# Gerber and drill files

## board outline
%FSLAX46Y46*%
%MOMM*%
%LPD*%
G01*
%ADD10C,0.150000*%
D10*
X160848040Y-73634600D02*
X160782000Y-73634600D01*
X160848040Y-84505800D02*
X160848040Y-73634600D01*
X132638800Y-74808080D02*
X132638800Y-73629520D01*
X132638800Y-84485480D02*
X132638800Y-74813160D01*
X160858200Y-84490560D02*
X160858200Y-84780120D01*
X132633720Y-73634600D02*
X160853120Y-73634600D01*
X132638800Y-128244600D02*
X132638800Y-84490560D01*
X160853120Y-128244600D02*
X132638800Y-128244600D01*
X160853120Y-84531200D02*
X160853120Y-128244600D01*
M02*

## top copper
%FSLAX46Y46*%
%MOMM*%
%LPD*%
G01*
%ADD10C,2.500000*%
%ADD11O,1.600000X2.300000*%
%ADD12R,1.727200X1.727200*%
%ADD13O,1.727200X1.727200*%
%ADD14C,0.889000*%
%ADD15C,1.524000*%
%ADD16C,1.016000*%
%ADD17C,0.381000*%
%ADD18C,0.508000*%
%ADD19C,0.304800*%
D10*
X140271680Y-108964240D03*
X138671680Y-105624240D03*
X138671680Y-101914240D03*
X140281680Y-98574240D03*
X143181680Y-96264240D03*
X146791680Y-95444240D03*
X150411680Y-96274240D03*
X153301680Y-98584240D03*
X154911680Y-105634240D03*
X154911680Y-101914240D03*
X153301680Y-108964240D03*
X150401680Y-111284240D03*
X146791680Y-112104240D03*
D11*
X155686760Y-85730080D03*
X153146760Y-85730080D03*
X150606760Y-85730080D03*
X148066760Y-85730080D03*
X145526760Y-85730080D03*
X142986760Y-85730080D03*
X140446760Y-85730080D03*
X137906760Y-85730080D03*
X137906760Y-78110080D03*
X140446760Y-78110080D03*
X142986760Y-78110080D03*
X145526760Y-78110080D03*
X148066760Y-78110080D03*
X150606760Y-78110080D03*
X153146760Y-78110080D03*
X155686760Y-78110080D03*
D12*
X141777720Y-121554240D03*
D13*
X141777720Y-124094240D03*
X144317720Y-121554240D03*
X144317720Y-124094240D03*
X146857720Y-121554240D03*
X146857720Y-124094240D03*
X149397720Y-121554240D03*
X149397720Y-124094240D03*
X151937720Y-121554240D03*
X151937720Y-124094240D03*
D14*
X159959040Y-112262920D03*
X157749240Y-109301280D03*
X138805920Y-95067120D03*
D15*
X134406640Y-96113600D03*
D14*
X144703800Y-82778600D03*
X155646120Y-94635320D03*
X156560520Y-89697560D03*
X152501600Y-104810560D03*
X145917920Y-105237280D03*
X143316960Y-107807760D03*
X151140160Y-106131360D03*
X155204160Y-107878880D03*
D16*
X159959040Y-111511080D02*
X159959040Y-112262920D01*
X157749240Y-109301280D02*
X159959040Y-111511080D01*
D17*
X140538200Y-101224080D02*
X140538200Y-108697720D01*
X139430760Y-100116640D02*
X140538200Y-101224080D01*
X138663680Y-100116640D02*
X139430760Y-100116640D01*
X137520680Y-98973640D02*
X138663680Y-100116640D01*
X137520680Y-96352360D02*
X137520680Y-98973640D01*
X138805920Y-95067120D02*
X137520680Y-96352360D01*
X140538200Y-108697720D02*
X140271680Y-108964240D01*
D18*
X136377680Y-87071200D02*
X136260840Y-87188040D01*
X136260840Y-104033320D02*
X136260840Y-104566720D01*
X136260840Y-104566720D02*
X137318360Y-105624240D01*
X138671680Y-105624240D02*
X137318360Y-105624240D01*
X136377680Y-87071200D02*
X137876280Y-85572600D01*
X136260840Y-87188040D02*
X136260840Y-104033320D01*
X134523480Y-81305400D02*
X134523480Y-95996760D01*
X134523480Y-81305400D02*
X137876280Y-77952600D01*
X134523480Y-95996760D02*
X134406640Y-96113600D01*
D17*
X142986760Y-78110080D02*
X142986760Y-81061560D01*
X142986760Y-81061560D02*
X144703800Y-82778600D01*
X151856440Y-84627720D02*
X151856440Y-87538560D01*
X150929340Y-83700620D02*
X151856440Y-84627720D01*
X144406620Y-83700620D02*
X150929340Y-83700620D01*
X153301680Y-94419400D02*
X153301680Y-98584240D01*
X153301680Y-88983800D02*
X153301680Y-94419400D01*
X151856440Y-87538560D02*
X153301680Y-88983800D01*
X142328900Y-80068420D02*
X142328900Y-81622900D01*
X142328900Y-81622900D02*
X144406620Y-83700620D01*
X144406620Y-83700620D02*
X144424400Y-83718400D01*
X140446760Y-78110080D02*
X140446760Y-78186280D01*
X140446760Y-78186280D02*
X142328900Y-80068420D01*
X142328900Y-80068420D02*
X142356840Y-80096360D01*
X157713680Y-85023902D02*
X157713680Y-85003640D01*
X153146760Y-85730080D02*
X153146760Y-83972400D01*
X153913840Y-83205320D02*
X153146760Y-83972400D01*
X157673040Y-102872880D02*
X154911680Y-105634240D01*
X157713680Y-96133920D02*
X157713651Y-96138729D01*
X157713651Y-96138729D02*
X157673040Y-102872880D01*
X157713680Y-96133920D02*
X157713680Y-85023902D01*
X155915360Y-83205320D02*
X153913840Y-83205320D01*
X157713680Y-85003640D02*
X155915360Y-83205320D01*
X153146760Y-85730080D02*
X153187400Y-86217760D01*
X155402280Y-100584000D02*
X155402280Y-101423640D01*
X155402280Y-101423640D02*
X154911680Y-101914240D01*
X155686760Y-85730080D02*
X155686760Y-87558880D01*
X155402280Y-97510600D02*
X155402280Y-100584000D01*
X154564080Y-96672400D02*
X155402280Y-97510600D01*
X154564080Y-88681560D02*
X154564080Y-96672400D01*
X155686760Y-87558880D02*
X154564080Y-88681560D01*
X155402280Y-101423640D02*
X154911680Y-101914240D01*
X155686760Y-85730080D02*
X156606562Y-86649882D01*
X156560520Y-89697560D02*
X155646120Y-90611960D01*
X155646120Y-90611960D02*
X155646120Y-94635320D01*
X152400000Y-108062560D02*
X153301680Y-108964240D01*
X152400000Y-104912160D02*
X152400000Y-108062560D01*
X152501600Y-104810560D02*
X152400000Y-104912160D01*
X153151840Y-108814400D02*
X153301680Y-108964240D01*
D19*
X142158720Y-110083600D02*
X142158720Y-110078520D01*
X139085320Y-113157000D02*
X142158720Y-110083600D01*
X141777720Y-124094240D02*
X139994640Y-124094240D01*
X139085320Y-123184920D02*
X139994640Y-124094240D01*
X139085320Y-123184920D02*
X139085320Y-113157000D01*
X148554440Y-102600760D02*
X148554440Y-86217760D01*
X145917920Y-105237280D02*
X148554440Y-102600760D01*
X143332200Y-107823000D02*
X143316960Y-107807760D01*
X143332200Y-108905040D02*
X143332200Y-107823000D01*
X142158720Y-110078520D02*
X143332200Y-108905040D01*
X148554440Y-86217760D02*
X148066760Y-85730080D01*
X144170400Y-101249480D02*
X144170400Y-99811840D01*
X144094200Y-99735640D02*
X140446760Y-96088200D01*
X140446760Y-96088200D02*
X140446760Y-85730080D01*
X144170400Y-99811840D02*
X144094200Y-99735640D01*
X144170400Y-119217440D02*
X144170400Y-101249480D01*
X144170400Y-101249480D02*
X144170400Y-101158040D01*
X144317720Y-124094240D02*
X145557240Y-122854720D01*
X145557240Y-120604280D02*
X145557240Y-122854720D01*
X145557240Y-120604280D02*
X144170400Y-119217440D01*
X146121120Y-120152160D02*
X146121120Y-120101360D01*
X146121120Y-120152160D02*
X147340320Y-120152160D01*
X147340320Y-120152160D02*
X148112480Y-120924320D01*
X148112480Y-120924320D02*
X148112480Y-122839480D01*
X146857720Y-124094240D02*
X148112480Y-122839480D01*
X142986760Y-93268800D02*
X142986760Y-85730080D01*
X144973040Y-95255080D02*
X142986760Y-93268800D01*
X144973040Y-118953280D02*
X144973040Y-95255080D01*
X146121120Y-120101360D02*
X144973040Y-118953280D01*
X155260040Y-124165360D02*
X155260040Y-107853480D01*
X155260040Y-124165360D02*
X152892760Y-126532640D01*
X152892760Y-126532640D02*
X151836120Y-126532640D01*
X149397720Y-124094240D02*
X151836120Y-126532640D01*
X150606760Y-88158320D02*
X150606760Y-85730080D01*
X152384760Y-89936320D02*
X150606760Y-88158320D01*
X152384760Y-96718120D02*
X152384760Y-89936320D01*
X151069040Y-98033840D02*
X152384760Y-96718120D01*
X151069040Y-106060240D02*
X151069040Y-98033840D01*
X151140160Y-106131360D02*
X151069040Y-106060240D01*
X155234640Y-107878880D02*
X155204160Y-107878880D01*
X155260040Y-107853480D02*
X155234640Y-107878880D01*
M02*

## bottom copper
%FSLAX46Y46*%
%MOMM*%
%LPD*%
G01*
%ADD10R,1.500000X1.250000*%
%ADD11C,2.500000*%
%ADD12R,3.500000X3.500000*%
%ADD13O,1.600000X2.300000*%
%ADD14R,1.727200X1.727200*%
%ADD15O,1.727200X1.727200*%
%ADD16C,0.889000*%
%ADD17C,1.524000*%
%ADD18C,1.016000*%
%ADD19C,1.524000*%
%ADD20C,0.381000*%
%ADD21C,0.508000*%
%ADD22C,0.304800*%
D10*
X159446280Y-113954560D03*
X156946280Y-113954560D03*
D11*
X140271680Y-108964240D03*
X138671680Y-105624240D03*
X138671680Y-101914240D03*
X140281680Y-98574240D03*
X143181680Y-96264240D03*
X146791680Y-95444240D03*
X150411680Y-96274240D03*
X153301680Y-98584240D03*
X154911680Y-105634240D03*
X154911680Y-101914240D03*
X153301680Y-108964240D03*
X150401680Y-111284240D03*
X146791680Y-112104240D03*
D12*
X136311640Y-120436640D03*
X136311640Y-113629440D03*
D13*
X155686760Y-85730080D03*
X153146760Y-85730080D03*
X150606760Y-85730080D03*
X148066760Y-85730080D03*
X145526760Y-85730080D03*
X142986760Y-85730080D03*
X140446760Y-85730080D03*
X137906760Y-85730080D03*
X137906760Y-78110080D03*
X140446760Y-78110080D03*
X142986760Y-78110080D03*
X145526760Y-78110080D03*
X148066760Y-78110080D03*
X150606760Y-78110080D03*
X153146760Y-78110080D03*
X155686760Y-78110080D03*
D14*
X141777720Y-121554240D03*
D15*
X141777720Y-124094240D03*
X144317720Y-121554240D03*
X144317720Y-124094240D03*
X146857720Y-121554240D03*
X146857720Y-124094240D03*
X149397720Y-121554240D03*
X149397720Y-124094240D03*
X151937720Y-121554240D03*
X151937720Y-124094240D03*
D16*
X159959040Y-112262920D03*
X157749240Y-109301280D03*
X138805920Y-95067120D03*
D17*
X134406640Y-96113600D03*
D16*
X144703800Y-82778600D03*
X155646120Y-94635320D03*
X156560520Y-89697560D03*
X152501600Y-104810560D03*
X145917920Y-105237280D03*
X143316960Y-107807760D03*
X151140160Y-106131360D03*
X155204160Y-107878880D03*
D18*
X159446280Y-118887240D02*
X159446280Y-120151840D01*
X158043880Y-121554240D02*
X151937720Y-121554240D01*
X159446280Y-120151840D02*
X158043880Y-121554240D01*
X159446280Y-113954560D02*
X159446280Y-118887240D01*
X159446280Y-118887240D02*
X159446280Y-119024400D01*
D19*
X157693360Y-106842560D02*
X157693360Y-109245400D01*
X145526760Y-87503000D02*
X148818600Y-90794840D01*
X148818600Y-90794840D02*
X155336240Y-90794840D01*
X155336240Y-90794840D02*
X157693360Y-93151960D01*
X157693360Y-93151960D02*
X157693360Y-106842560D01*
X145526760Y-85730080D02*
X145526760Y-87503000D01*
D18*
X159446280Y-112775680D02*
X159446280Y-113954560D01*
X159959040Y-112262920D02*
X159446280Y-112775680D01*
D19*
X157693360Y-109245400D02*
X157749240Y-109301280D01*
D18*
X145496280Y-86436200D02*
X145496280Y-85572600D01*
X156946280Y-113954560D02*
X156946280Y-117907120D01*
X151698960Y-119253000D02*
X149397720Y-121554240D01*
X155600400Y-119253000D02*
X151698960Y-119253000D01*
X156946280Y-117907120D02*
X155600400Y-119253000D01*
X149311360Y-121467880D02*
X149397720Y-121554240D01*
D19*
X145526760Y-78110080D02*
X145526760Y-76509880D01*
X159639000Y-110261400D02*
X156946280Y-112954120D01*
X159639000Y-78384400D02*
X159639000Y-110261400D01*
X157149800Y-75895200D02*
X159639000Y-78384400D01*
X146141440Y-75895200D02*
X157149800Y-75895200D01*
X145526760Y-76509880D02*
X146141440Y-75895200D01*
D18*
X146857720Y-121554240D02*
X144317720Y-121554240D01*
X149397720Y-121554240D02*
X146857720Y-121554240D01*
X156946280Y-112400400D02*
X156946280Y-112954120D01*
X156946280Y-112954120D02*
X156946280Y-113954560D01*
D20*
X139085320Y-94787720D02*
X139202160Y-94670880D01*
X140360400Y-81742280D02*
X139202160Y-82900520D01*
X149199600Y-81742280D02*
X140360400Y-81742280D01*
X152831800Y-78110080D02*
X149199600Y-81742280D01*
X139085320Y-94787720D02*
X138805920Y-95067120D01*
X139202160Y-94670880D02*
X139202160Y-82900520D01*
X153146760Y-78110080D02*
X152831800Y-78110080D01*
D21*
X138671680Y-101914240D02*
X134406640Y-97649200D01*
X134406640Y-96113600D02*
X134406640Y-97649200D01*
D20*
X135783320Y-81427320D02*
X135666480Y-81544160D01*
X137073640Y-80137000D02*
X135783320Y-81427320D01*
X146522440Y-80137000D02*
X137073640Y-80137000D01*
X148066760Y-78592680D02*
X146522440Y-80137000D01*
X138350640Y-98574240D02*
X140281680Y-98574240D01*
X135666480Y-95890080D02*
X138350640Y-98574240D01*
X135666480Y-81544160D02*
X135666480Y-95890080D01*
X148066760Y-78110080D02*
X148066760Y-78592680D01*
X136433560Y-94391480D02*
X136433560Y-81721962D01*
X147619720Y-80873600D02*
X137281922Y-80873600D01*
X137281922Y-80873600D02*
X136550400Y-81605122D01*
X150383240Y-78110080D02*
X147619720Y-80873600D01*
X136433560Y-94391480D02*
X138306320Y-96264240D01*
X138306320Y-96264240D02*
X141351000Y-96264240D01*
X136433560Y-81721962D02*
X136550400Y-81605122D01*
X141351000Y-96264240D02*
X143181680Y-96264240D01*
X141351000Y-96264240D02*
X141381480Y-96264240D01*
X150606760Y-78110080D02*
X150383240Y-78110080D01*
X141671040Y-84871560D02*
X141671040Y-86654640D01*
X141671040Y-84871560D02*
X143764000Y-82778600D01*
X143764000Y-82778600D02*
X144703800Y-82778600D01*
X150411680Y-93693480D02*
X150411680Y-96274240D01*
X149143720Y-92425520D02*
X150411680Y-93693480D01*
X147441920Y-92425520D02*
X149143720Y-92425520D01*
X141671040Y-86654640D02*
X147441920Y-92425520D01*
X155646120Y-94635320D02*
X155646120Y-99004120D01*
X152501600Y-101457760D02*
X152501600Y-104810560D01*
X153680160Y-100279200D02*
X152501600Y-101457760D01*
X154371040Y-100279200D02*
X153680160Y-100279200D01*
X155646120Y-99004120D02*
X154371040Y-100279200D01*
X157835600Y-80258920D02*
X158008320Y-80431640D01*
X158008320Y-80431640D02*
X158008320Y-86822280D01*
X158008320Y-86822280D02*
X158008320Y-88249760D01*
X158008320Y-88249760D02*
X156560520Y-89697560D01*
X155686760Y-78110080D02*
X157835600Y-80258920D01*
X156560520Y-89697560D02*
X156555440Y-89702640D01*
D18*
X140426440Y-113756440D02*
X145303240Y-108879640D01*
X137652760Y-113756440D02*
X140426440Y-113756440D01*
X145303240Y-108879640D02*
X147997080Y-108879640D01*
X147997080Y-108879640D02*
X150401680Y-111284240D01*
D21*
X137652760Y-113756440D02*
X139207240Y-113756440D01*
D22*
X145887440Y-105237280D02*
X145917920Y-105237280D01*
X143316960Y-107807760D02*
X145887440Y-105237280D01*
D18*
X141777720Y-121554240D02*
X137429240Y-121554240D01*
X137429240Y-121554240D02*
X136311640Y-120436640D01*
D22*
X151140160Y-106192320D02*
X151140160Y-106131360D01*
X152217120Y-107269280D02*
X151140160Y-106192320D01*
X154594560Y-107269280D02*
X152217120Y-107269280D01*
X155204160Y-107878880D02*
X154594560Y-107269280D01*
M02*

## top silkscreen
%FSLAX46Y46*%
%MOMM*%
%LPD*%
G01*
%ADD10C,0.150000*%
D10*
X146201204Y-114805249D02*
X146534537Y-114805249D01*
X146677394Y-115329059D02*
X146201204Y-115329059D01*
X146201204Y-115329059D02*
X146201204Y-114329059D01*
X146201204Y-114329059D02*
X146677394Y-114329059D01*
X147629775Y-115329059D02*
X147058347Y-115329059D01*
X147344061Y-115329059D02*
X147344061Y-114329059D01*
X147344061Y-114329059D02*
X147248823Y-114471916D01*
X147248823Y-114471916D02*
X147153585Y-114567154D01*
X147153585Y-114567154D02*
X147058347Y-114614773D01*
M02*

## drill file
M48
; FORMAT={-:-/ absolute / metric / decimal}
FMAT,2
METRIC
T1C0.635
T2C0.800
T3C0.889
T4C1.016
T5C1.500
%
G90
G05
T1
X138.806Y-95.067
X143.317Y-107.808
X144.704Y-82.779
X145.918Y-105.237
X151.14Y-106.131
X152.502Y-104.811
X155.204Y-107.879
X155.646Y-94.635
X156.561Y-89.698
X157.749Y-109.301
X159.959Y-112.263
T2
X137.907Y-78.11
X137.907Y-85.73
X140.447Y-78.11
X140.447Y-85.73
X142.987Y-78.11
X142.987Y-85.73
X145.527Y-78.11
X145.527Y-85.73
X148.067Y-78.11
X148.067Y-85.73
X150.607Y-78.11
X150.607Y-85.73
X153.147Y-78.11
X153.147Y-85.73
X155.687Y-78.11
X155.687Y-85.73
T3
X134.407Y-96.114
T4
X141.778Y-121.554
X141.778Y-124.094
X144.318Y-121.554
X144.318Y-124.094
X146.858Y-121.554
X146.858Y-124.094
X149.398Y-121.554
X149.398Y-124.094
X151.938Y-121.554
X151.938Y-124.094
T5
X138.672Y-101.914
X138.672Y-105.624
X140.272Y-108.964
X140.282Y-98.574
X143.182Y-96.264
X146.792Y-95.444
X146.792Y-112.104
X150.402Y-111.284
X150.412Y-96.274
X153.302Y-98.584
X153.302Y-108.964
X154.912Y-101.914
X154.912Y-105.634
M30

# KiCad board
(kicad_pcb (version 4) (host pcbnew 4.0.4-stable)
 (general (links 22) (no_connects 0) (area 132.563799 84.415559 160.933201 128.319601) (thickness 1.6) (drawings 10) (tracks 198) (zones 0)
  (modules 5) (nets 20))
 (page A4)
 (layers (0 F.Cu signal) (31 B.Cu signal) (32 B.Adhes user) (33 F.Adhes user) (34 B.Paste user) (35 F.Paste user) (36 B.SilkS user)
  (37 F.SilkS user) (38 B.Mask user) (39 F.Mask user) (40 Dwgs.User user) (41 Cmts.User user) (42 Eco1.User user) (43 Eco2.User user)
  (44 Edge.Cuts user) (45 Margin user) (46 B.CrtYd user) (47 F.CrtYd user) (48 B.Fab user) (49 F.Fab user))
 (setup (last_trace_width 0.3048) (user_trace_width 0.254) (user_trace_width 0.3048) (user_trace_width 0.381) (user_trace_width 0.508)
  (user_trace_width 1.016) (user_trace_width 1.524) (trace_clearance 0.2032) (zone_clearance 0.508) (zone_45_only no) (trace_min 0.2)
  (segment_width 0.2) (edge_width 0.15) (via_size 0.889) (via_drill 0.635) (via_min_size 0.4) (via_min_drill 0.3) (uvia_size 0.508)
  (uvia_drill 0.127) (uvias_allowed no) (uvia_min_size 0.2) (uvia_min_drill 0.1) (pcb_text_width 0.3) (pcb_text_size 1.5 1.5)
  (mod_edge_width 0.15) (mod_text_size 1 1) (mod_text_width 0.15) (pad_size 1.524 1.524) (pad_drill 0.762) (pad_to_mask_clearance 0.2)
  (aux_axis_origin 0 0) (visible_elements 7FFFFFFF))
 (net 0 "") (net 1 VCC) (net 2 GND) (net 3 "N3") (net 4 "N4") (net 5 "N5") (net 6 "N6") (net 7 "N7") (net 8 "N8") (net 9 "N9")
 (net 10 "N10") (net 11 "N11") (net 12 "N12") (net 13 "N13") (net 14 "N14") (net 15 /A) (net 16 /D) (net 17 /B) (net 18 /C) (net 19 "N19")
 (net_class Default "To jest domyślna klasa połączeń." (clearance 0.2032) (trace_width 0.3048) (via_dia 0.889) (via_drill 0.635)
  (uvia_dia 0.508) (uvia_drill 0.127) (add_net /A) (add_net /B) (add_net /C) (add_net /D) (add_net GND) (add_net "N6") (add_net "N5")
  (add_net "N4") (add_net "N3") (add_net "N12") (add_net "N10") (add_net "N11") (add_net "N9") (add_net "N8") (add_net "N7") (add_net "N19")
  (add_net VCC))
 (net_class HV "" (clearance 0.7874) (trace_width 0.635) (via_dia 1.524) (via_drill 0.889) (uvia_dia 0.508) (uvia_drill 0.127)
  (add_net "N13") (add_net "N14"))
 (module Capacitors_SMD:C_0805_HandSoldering (layer B.Cu) (at 158.19628 113.95456 180)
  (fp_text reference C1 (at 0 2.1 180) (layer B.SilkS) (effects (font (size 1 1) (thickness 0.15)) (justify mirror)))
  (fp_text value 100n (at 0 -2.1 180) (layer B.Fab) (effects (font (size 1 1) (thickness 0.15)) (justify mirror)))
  (pad 1 smd rect (at -1.25 0 180) (size 1.5 1.25) (layers B.Cu B.Paste B.Mask) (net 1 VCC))
  (pad 2 smd rect (at 1.25 0 180) (size 1.5 1.25) (layers B.Cu B.Paste B.Mask) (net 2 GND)))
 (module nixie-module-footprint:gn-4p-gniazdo (layer F.Cu) (at 146.79168 103.77424)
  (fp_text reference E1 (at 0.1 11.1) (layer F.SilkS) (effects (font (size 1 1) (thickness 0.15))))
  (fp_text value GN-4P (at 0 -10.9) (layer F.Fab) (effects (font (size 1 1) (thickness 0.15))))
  (pad 13 thru_hole circle (at -6.52 5.19) (size 2.5 2.5) (drill 1.5) (layers *.Cu *.Mask) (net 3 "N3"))
  (pad 12 thru_hole circle (at -8.12 1.85) (size 2.5 2.5) (drill 1.5) (layers *.Cu *.Mask) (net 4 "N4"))
  (pad 11 thru_hole circle (at -8.12 -1.86) (size 2.5 2.5) (drill 1.5) (layers *.Cu *.Mask) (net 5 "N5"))
  (pad 10 thru_hole circle (at -6.51 -5.2) (size 2.5 2.5) (drill 1.5) (layers *.Cu *.Mask) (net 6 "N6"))
  (pad 9 thru_hole circle (at -3.61 -7.51) (size 2.5 2.5) (drill 1.5) (layers *.Cu *.Mask) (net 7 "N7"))
  (pad 8 thru_hole circle (at 0 -8.33) (size 2.5 2.5) (drill 1.5) (layers *.Cu *.Mask))
  (pad 7 thru_hole circle (at 3.62 -7.5) (size 2.5 2.5) (drill 1.5) (layers *.Cu *.Mask) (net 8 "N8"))
  (pad 6 thru_hole circle (at 6.51 -5.19) (size 2.5 2.5) (drill 1.5) (layers *.Cu *.Mask) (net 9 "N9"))
  (pad 4 thru_hole circle (at 8.12 1.86) (size 2.5 2.5) (drill 1.5) (layers *.Cu *.Mask) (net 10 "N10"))
  (pad 5 thru_hole circle (at 8.12 -1.86) (size 2.5 2.5) (drill 1.5) (layers *.Cu *.Mask) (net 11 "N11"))
  (pad 3 thru_hole circle (at 6.51 5.19) (size 2.5 2.5) (drill 1.5) (layers *.Cu *.Mask) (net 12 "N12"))
  (pad 2 thru_hole circle (at 3.61 7.51) (size 2.5 2.5) (drill 1.5) (layers *.Cu *.Mask) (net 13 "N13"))
  (pad 1 thru_hole circle (at 0 8.33 25.71) (size 2.5 2.5) (drill 1.5) (layers *.Cu *.Mask)))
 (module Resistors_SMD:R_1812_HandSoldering (layer B.Cu) (at 136.31164 117.03304 90)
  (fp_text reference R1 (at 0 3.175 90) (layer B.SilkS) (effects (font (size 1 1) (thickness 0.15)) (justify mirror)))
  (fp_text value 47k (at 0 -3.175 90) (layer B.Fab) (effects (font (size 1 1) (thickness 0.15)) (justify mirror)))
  (pad 1 smd rect (at -3.4036 0 90) (size 3.5 3.5) (layers B.Cu B.Paste B.Mask) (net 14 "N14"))
  (pad 2 smd rect (at 3.4036 0 90) (size 3.5 3.5) (layers B.Cu B.Paste B.Mask) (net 13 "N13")))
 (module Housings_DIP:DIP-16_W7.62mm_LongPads (layer B.Cu) (at 155.68676 85.73008 90)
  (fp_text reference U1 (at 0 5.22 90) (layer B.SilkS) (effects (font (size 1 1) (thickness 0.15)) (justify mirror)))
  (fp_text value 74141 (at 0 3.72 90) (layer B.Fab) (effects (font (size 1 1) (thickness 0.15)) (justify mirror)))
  (pad 1 thru_hole oval (at 0 0 90) (size 2.3 1.6) (drill 0.8) (layers *.Cu *.Mask) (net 11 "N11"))
  (pad 2 thru_hole oval (at 0 -2.54 90) (size 2.3 1.6) (drill 0.8) (layers *.Cu *.Mask) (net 10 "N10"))
  (pad 3 thru_hole oval (at 0 -5.08 90) (size 2.3 1.6) (drill 0.8) (layers *.Cu *.Mask) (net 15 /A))
  (pad 4 thru_hole oval (at 0 -7.62 90) (size 2.3 1.6) (drill 0.8) (layers *.Cu *.Mask) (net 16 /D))
  (pad 5 thru_hole oval (at 0 -10.16 90) (size 2.3 1.6) (drill 0.8) (layers *.Cu *.Mask) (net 1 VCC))
  (pad 6 thru_hole oval (at 0 -12.7 90) (size 2.3 1.6) (drill 0.8) (layers *.Cu *.Mask) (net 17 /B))
  (pad 7 thru_hole oval (at 0 -15.24 90) (size 2.3 1.6) (drill 0.8) (layers *.Cu *.Mask) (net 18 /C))
  (pad 8 thru_hole oval (at 0 -17.78 90) (size 2.3 1.6) (drill 0.8) (layers *.Cu *.Mask) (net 4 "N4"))
  (pad 9 thru_hole oval (at 7.62 -17.78 90) (size 2.3 1.6) (drill 0.8) (layers *.Cu *.Mask) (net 5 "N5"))
  (pad 10 thru_hole oval (at 7.62 -15.24 90) (size 2.3 1.6) (drill 0.8) (layers *.Cu *.Mask) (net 9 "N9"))
  (pad 11 thru_hole oval (at 7.62 -12.7 90) (size 2.3 1.6) (drill 0.8) (layers *.Cu *.Mask) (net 8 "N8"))
  (pad 12 thru_hole oval (at 7.62 -10.16 90) (size 2.3 1.6) (drill 0.8) (layers *.Cu *.Mask) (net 2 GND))
  (pad 13 thru_hole oval (at 7.62 -7.62 90) (size 2.3 1.6) (drill 0.8) (layers *.Cu *.Mask) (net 6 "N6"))
  (pad 14 thru_hole oval (at 7.62 -5.08 90) (size 2.3 1.6) (drill 0.8) (layers *.Cu *.Mask) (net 7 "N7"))
  (pad 15 thru_hole oval (at 7.62 -2.54 90) (size 2.3 1.6) (drill 0.8) (layers *.Cu *.Mask) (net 3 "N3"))
  (pad 16 thru_hole oval (at 7.62 0 90) (size 2.3 1.6) (drill 0.8) (layers *.Cu *.Mask) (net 12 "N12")))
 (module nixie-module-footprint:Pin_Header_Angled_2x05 (layer B.Cu) (at 141.77772 121.55424 270)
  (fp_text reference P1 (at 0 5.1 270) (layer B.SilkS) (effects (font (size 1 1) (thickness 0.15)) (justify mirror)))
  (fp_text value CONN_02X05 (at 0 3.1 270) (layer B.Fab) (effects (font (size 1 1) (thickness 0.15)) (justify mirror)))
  (pad 2 thru_hole rect (at 0 0 270) (size 1.7272 1.7272) (drill 1.016) (layers *.Cu *.Mask) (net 14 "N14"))
  (pad 1 thru_hole oval (at 2.54 0 270) (size 1.7272 1.7272) (drill 1.016) (layers *.Cu *.Mask) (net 16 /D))
  (pad 4 thru_hole oval (at 0 -2.54 270) (size 1.7272 1.7272) (drill 1.016) (layers *.Cu *.Mask) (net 2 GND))
  (pad 3 thru_hole oval (at 2.54 -2.54 270) (size 1.7272 1.7272) (drill 1.016) (layers *.Cu *.Mask) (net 18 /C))
  (pad 6 thru_hole oval (at 0 -5.08 270) (size 1.7272 1.7272) (drill 1.016) (layers *.Cu *.Mask) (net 2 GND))
  (pad 5 thru_hole oval (at 2.54 -5.08 270) (size 1.7272 1.7272) (drill 1.016) (layers *.Cu *.Mask) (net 17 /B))
  (pad 8 thru_hole oval (at 0 -7.62 270) (size 1.7272 1.7272) (drill 1.016) (layers *.Cu *.Mask) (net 2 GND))
  (pad 7 thru_hole oval (at 2.54 -7.62 270) (size 1.7272 1.7272) (drill 1.016) (layers *.Cu *.Mask) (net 15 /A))
  (pad 10 thru_hole oval (at 0 -10.16 270) (size 1.7272 1.7272) (drill 1.016) (layers *.Cu *.Mask) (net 1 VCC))
  (pad 9 thru_hole oval (at 2.54 -10.16 270) (size 1.7272 1.7272) (drill 1.016) (layers *.Cu *.Mask) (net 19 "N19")))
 (gr_line (start 160.84804 73.6346) (end 160.782 73.6346) (angle 90) (layer Edge.Cuts) (width 0.15))
 (gr_line (start 160.84804 84.5058) (end 160.84804 73.6346) (angle 90) (layer Edge.Cuts) (width 0.15))
 (gr_line (start 132.6388 74.80808) (end 132.6388 73.62952) (angle 90) (layer Edge.Cuts) (width 0.15))
 (gr_line (start 132.6388 84.48548) (end 132.6388 74.81316) (angle 90) (layer Edge.Cuts) (width 0.15))
 (gr_line (start 160.8582 84.49056) (end 160.8582 84.78012) (angle 90) (layer Edge.Cuts) (width 0.15))
 (gr_line (start 132.63372 73.6346) (end 160.85312 73.6346) (angle 90) (layer Edge.Cuts) (width 0.15))
 (gr_line (start 132.6388 128.2446) (end 132.6388 84.49056) (angle 90) (layer Edge.Cuts) (width 0.15))
 (gr_line (start 160.85312 128.2446) (end 132.6388 128.2446) (angle 90) (layer Edge.Cuts) (width 0.15))
 (gr_line (start 160.85312 84.5312) (end 160.85312 128.2446) (angle 90) (layer Edge.Cuts) (width 0.15))
 (segment (start 159.44628 118.88724) (end 159.44628 120.15184) (width 1.016) (layer B.Cu) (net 1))
 (segment (start 158.04388 121.55424) (end 151.93772 121.55424) (width 1.016) (layer B.Cu) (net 1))
 (segment (start 159.44628 120.15184) (end 158.04388 121.55424) (width 1.016) (layer B.Cu) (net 1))
 (segment (start 159.44628 113.95456) (end 159.44628 118.88724) (width 1.016) (layer B.Cu) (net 1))
 (segment (start 159.44628 118.88724) (end 159.44628 119.0244) (width 1.016) (layer B.Cu) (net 1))
 (segment (start 157.69336 106.84256) (end 157.69336 109.2454) (width 1.524) (layer B.Cu) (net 1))
 (segment (start 145.52676 87.503) (end 148.8186 90.79484) (width 1.524) (layer B.Cu) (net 1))
 (segment (start 148.8186 90.79484) (end 155.33624 90.79484) (width 1.524) (layer B.Cu) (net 1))
 (segment (start 155.33624 90.79484) (end 157.69336 93.15196) (width 1.524) (layer B.Cu) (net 1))
 (segment (start 157.69336 93.15196) (end 157.69336 106.84256) (width 1.524) (layer B.Cu) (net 1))
 (segment (start 145.52676 85.73008) (end 145.52676 87.503) (width 1.524) (layer B.Cu) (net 1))
 (segment (start 159.44628 112.77568) (end 159.44628 113.95456) (width 1.016) (layer B.Cu) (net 1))
 (segment (start 159.95904 112.26292) (end 159.44628 112.77568) (width 1.016) (layer B.Cu) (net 1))
 (via (at 159.95904 112.26292) (size 0.889) (drill 0.635) (layers F.Cu B.Cu) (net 1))
 (segment (start 159.95904 111.51108) (end 159.95904 112.26292) (width 1.016) (layer F.Cu) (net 1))
 (segment (start 157.74924 109.30128) (end 159.95904 111.51108) (width 1.016) (layer F.Cu) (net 1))
 (via (at 157.74924 109.30128) (size 0.889) (drill 0.635) (layers F.Cu B.Cu) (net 1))
 (segment (start 157.69336 109.2454) (end 157.74924 109.30128) (width 1.524) (layer B.Cu) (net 1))
 (segment (start 145.49628 86.4362) (end 145.49628 85.5726) (width 1.016) (layer B.Cu) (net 1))
 (segment (start 156.94628 113.95456) (end 156.94628 117.90712) (width 1.016) (layer B.Cu) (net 2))
 (segment (start 151.69896 119.253) (end 149.39772 121.55424) (width 1.016) (layer B.Cu) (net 2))
 (segment (start 155.6004 119.253) (end 151.69896 119.253) (width 1.016) (layer B.Cu) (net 2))
 (segment (start 156.94628 117.90712) (end 155.6004 119.253) (width 1.016) (layer B.Cu) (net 2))
 (segment (start 149.31136 121.46788) (end 149.39772 121.55424) (width 1.016) (layer B.Cu) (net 2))
 (segment (start 145.52676 78.11008) (end 145.52676 76.50988) (width 1.524) (layer B.Cu) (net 2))
 (segment (start 159.639 110.2614) (end 156.94628 112.95412) (width 1.524) (layer B.Cu) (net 2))
 (segment (start 159.639 78.3844) (end 159.639 110.2614) (width 1.524) (layer B.Cu) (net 2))
 (segment (start 157.1498 75.8952) (end 159.639 78.3844) (width 1.524) (layer B.Cu) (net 2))
 (segment (start 146.14144 75.8952) (end 157.1498 75.8952) (width 1.524) (layer B.Cu) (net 2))
 (segment (start 145.52676 76.50988) (end 146.14144 75.8952) (width 1.524) (layer B.Cu) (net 2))
 (segment (start 146.85772 121.55424) (end 144.31772 121.55424) (width 1.016) (layer B.Cu) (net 2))
 (segment (start 149.39772 121.55424) (end 146.85772 121.55424) (width 1.016) (layer B.Cu) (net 2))
 (segment (start 156.94628 112.4004) (end 156.94628 112.95412) (width 1.016) (layer B.Cu) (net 2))
 (segment (start 156.94628 112.95412) (end 156.94628 113.95456) (width 1.016) (layer B.Cu) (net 2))
 (segment (start 139.08532 94.78772) (end 139.20216 94.67088) (width 0.381) (layer B.Cu) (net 3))
 (segment (start 140.3604 81.74228) (end 139.20216 82.90052) (width 0.381) (layer B.Cu) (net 3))
 (segment (start 149.1996 81.74228) (end 140.3604 81.74228) (width 0.381) (layer B.Cu) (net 3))
 (segment (start 152.8318 78.11008) (end 149.1996 81.74228) (width 0.381) (layer B.Cu) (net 3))
 (segment (start 140.5382 101.22408) (end 140.5382 108.69772) (width 0.381) (layer F.Cu) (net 3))
 (segment (start 139.43076 100.11664) (end 140.5382 101.22408) (width 0.381) (layer F.Cu) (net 3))
 (segment (start 138.66368 100.11664) (end 139.43076 100.11664) (width 0.381) (layer F.Cu) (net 3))
 (segment (start 137.52068 98.97364) (end 138.66368 100.11664) (width 0.381) (layer F.Cu) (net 3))
 (segment (start 137.52068 96.35236) (end 137.52068 98.97364) (width 0.381) (layer F.Cu) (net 3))
 (segment (start 138.80592 95.06712) (end 137.52068 96.35236) (width 0.381) (layer F.Cu) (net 3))
 (via (at 138.80592 95.06712) (size 0.889) (drill 0.635) (layers F.Cu B.Cu) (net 3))
 (segment (start 139.08532 94.78772) (end 138.80592 95.06712) (width 0.381) (layer B.Cu) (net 3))
 (segment (start 139.20216 94.67088) (end 139.20216 82.90052) (width 0.381) (layer B.Cu) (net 3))
 (segment (start 140.5382 108.69772) (end 140.27168 108.96424) (width 0.381) (layer F.Cu) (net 3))
 (segment (start 153.14676 78.11008) (end 152.8318 78.11008) (width 0.381) (layer B.Cu) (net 3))
 (segment (start 136.37768 87.0712) (end 136.26084 87.18804) (width 0.508) (layer F.Cu) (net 4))
 (segment (start 136.26084 104.03332) (end 136.26084 104.56672) (width 0.508) (layer F.Cu) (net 4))
 (segment (start 136.26084 104.56672) (end 137.31836 105.62424) (width 0.508) (layer F.Cu) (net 4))
 (segment (start 138.67168 105.62424) (end 137.31836 105.62424) (width 0.508) (layer F.Cu) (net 4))
 (segment (start 136.37768 87.0712) (end 137.87628 85.5726) (width 0.508) (layer F.Cu) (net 4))
 (segment (start 136.26084 87.18804) (end 136.26084 104.03332) (width 0.508) (layer F.Cu) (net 4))
 (segment (start 134.52348 81.3054) (end 134.52348 95.99676) (width 0.508) (layer F.Cu) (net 5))
 (segment (start 138.67168 101.91424) (end 134.40664 97.6492) (width 0.508) (layer B.Cu) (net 5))
 (segment (start 134.40664 96.1136) (end 134.40664 97.6492) (width 0.508) (layer B.Cu) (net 5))
 (via (at 134.40664 96.1136) (size 1.524) (drill 0.889) (layers F.Cu B.Cu) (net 5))
 (segment (start 134.52348 81.3054) (end 137.87628 77.9526) (width 0.508) (layer F.Cu) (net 5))
 (segment (start 134.52348 95.99676) (end 134.40664 96.1136) (width 0.508) (layer F.Cu) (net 5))
 (segment (start 135.78332 81.42732) (end 135.66648 81.54416) (width 0.381) (layer B.Cu) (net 6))
 (segment (start 137.07364 80.137) (end 135.78332 81.42732) (width 0.381) (layer B.Cu) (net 6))
 (segment (start 146.52244 80.137) (end 137.07364 80.137) (width 0.381) (layer B.Cu) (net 6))
 (segment (start 148.06676 78.59268) (end 146.52244 80.137) (width 0.381) (layer B.Cu) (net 6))
 (segment (start 138.35064 98.57424) (end 140.28168 98.57424) (width 0.381) (layer B.Cu) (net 6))
 (segment (start 135.66648 95.89008) (end 138.35064 98.57424) (width 0.381) (layer B.Cu) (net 6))
 (segment (start 135.66648 81.54416) (end 135.66648 95.89008) (width 0.381) (layer B.Cu) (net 6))
 (segment (start 148.06676 78.11008) (end 148.06676 78.59268) (width 0.381) (layer B.Cu) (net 6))
 (segment (start 136.43356 94.39148) (end 136.43356 81.721962) (width 0.381) (layer B.Cu) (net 7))
 (segment (start 147.61972 80.8736) (end 137.281922 80.8736) (width 0.381) (layer B.Cu) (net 7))
 (segment (start 137.281922 80.8736) (end 136.5504 81.605122) (width 0.381) (layer B.Cu) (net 7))
 (segment (start 150.38324 78.11008) (end 147.61972 80.8736) (width 0.381) (layer B.Cu) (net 7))
 (segment (start 136.43356 94.39148) (end 138.30632 96.26424) (width 0.381) (layer B.Cu) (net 7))
 (segment (start 138.30632 96.26424) (end 141.351 96.26424) (width 0.381) (layer B.Cu) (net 7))
 (segment (start 136.43356 81.721962) (end 136.5504 81.605122) (width 0.381) (layer B.Cu) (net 7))
 (segment (start 141.351 96.26424) (end 143.18168 96.26424) (width 0.381) (layer B.Cu) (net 7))
 (segment (start 141.351 96.26424) (end 141.38148 96.26424) (width 0.381) (layer B.Cu) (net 7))
 (segment (start 150.60676 78.11008) (end 150.38324 78.11008) (width 0.381) (layer B.Cu) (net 7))
 (segment (start 141.67104 84.87156) (end 141.67104 86.65464) (width 0.381) (layer B.Cu) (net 8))
 (segment (start 142.98676 78.11008) (end 142.98676 81.06156) (width 0.381) (layer F.Cu) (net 8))
 (via (at 144.7038 82.7786) (size 0.889) (drill 0.635) (layers F.Cu B.Cu) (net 8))
 (segment (start 142.98676 81.06156) (end 144.7038 82.7786) (width 0.381) (layer F.Cu) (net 8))
 (segment (start 141.67104 84.87156) (end 143.764 82.7786) (width 0.381) (layer B.Cu) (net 8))
 (segment (start 143.764 82.7786) (end 144.7038 82.7786) (width 0.381) (layer B.Cu) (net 8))
 (segment (start 150.41168 93.69348) (end 150.41168 96.27424) (width 0.381) (layer B.Cu) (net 8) (status 800000))
 (segment (start 149.14372 92.42552) (end 150.41168 93.69348) (width 0.381) (layer B.Cu) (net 8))
 (segment (start 147.44192 92.42552) (end 149.14372 92.42552) (width 0.381) (layer B.Cu) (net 8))
 (segment (start 141.67104 86.65464) (end 147.44192 92.42552) (width 0.381) (layer B.Cu) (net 8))
 (segment (start 151.85644 84.62772) (end 151.85644 87.53856) (width 0.381) (layer F.Cu) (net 9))
 (segment (start 150.92934 83.70062) (end 151.85644 84.62772) (width 0.381) (layer F.Cu) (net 9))
 (segment (start 144.40662 83.70062) (end 150.92934 83.70062) (width 0.381) (layer F.Cu) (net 9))
 (segment (start 153.30168 94.4194) (end 153.30168 98.58424) (width 0.381) (layer F.Cu) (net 9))
 (segment (start 153.30168 88.9838) (end 153.30168 94.4194) (width 0.381) (layer F.Cu) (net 9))
 (segment (start 151.85644 87.53856) (end 153.30168 88.9838) (width 0.381) (layer F.Cu) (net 9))
 (segment (start 142.3289 80.06842) (end 142.3289 81.6229) (width 0.381) (layer F.Cu) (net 9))
 (segment (start 142.3289 81.6229) (end 144.40662 83.70062) (width 0.381) (layer F.Cu) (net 9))
 (segment (start 144.40662 83.70062) (end 144.4244 83.7184) (width 0.381) (layer F.Cu) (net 9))
 (segment (start 140.44676 78.11008) (end 140.44676 78.18628) (width 0.381) (layer F.Cu) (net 9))
 (segment (start 140.44676 78.18628) (end 142.3289 80.06842) (width 0.381) (layer F.Cu) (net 9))
 (segment (start 142.3289 80.06842) (end 142.35684 80.09636) (width 0.381) (layer F.Cu) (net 9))
 (segment (start 157.71368 85.023902) (end 157.71368 85.00364) (width 0.381) (layer F.Cu) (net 10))
 (segment (start 153.14676 85.73008) (end 153.14676 83.9724) (width 0.381) (layer F.Cu) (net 10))
 (segment (start 153.91384 83.20532) (end 153.14676 83.9724) (width 0.381) (layer F.Cu) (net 10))
 (segment (start 157.67304 102.87288) (end 154.91168 105.63424) (width 0.381) (layer F.Cu) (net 10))
 (segment (start 157.71368 96.13392) (end 157.713651 96.138729) (width 0.381) (layer F.Cu) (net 10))
 (segment (start 157.713651 96.138729) (end 157.67304 102.87288) (width 0.381) (layer F.Cu) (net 10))
 (segment (start 157.71368 96.13392) (end 157.71368 85.023902) (width 0.381) (layer F.Cu) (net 10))
 (segment (start 155.91536 83.20532) (end 153.91384 83.20532) (width 0.381) (layer F.Cu) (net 10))
 (segment (start 157.71368 85.00364) (end 155.91536 83.20532) (width 0.381) (layer F.Cu) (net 10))
 (segment (start 153.14676 85.73008) (end 153.1874 86.21776) (width 0.381) (layer F.Cu) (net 10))
 (segment (start 155.40228 100.584) (end 155.40228 101.42364) (width 0.381) (layer F.Cu) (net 11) (status 800000))
 (segment (start 155.40228 101.42364) (end 154.91168 101.91424) (width 0.381) (layer F.Cu) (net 11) (status C00000))
 (segment (start 155.68676 85.73008) (end 155.68676 87.55888) (width 0.381) (layer F.Cu) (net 11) (status 400000))
 (segment (start 155.40228 97.5106) (end 155.40228 100.584) (width 0.381) (layer F.Cu) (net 11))
 (segment (start 154.56408 96.6724) (end 155.40228 97.5106) (width 0.381) (layer F.Cu) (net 11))
 (segment (start 154.56408 88.68156) (end 154.56408 96.6724) (width 0.381) (layer F.Cu) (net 11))
 (segment (start 155.68676 87.55888) (end 154.56408 88.68156) (width 0.381) (layer F.Cu) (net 11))
 (segment (start 155.40228 101.42364) (end 154.91168 101.91424) (width 0.381) (layer F.Cu) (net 11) (status C00000))
 (segment (start 155.68676 85.73008) (end 156.606562 86.649882) (width 0.381) (layer F.Cu) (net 11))
 (segment (start 155.64612 94.63532) (end 155.64612 99.00412) (width 0.381) (layer B.Cu) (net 12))
 (segment (start 156.56052 89.69756) (end 155.64612 90.61196) (width 0.381) (layer F.Cu) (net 12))
 (segment (start 155.64612 90.61196) (end 155.64612 94.63532) (width 0.381) (layer F.Cu) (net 12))
 (via (at 155.64612 94.63532) (size 0.889) (drill 0.635) (layers F.Cu B.Cu) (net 12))
 (via (at 156.56052 89.69756) (size 0.889) (drill 0.635) (layers F.Cu B.Cu) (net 12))
 (segment (start 152.4 108.06256) (end 153.30168 108.96424) (width 0.381) (layer F.Cu) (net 12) (status 800000))
 (segment (start 152.4 104.91216) (end 152.4 108.06256) (width 0.381) (layer F.Cu) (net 12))
 (segment (start 152.5016 104.81056) (end 152.4 104.91216) (width 0.381) (layer F.Cu) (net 12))
 (via (at 152.5016 104.81056) (size 0.889) (drill 0.635) (layers F.Cu B.Cu) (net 12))
 (segment (start 152.5016 101.45776) (end 152.5016 104.81056) (width 0.381) (layer B.Cu) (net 12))
 (segment (start 153.68016 100.2792) (end 152.5016 101.45776) (width 0.381) (layer B.Cu) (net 12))
 (segment (start 154.37104 100.2792) (end 153.68016 100.2792) (width 0.381) (layer B.Cu) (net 12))
 (segment (start 155.64612 99.00412) (end 154.37104 100.2792) (width 0.381) (layer B.Cu) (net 12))
 (segment (start 157.8356 80.25892) (end 158.00832 80.43164) (width 0.381) (layer B.Cu) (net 12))
 (segment (start 158.00832 80.43164) (end 158.00832 86.82228) (width 0.381) (layer B.Cu) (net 12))
 (segment (start 158.00832 86.82228) (end 158.00832 88.24976) (width 0.381) (layer B.Cu) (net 12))
 (segment (start 158.00832 88.24976) (end 156.56052 89.69756) (width 0.381) (layer B.Cu) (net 12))
 (segment (start 155.68676 78.11008) (end 157.8356 80.25892) (width 0.381) (layer B.Cu) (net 12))
 (segment (start 156.56052 89.69756) (end 156.55544 89.70264) (width 0.381) (layer B.Cu) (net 12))
 (segment (start 153.15184 108.8144) (end 153.30168 108.96424) (width 0.381) (layer F.Cu) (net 12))
 (segment (start 140.42644 113.75644) (end 145.30324 108.87964) (width 1.016) (layer B.Cu) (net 13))
 (segment (start 137.65276 113.75644) (end 140.42644 113.75644) (width 1.016) (layer B.Cu) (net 13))
 (segment (start 145.30324 108.87964) (end 147.99708 108.87964) (width 1.016) (layer B.Cu) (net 13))
 (segment (start 147.99708 108.87964) (end 150.40168 111.28424) (width 1.016) (layer B.Cu) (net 13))
 (segment (start 137.65276 113.75644) (end 139.20724 113.75644) (width 0.508) (layer B.Cu) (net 13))
 (segment (start 142.15872 110.0836) (end 142.15872 110.07852) (width 0.3048) (layer F.Cu) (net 16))
 (segment (start 139.08532 113.157) (end 142.15872 110.0836) (width 0.3048) (layer F.Cu) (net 16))
 (segment (start 141.77772 124.09424) (end 139.99464 124.09424) (width 0.3048) (layer F.Cu) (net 16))
 (segment (start 139.08532 123.18492) (end 139.99464 124.09424) (width 0.3048) (layer F.Cu) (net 16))
 (segment (start 139.08532 123.18492) (end 139.08532 113.157) (width 0.3048) (layer F.Cu) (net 16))
 (segment (start 148.55444 102.60076) (end 148.55444 86.21776) (width 0.3048) (layer F.Cu) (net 16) (status 800000))
 (segment (start 145.91792 105.23728) (end 148.55444 102.60076) (width 0.3048) (layer F.Cu) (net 16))
 (via (at 145.91792 105.23728) (size 0.889) (drill 0.635) (layers F.Cu B.Cu) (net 16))
 (segment (start 145.88744 105.23728) (end 145.91792 105.23728) (width 0.3048) (layer B.Cu) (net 16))
 (segment (start 143.31696 107.80776) (end 145.88744 105.23728) (width 0.3048) (layer B.Cu) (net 16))
 (via (at 143.31696 107.80776) (size 0.889) (drill 0.635) (layers F.Cu B.Cu) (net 16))
 (segment (start 143.3322 107.823) (end 143.31696 107.80776) (width 0.3048) (layer F.Cu) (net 16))
 (segment (start 143.3322 108.90504) (end 143.3322 107.823) (width 0.3048) (layer F.Cu) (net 16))
 (segment (start 142.15872 110.07852) (end 143.3322 108.90504) (width 0.3048) (layer F.Cu) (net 16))
 (segment (start 148.55444 86.21776) (end 148.06676 85.73008) (width 0.3048) (layer F.Cu) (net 16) (status C00000))
 (segment (start 141.77772 121.55424) (end 137.42924 121.55424) (width 1.016) (layer B.Cu) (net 14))
 (segment (start 137.42924 121.55424) (end 136.31164 120.43664) (width 1.016) (layer B.Cu) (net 14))
 (segment (start 144.1704 101.24948) (end 144.1704 99.81184) (width 0.3048) (layer F.Cu) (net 18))
 (segment (start 144.0942 99.73564) (end 140.44676 96.0882) (width 0.3048) (layer F.Cu) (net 18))
 (segment (start 140.44676 96.0882) (end 140.44676 85.73008) (width 0.3048) (layer F.Cu) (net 18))
 (segment (start 144.1704 99.81184) (end 144.0942 99.73564) (width 0.3048) (layer F.Cu) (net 18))
 (segment (start 144.1704 119.21744) (end 144.1704 101.24948) (width 0.3048) (layer F.Cu) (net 18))
 (segment (start 144.1704 101.24948) (end 144.1704 101.15804) (width 0.3048) (layer F.Cu) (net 18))
 (segment (start 144.31772 124.09424) (end 145.55724 122.85472) (width 0.3048) (layer F.Cu) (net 18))
 (segment (start 145.55724 120.60428) (end 145.55724 122.85472) (width 0.3048) (layer F.Cu) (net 18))
 (segment (start 145.55724 120.60428) (end 144.1704 119.21744) (width 0.3048) (layer F.Cu) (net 18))
 (segment (start 146.12112 120.15216) (end 146.12112 120.10136) (width 0.3048) (layer F.Cu) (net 17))
 (segment (start 146.12112 120.15216) (end 147.34032 120.15216) (width 0.3048) (layer F.Cu) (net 17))
 (segment (start 147.34032 120.15216) (end 148.11248 120.92432) (width 0.3048) (layer F.Cu) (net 17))
 (segment (start 148.11248 120.92432) (end 148.11248 122.83948) (width 0.3048) (layer F.Cu) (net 17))
 (segment (start 146.85772 124.09424) (end 148.11248 122.83948) (width 0.3048) (layer F.Cu) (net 17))
 (segment (start 142.98676 93.2688) (end 142.98676 85.73008) (width 0.3048) (layer F.Cu) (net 17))
 (segment (start 144.97304 95.25508) (end 142.98676 93.2688) (width 0.3048) (layer F.Cu) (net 17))
 (segment (start 144.97304 118.95328) (end 144.97304 95.25508) (width 0.3048) (layer F.Cu) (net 17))
 (segment (start 146.12112 120.10136) (end 144.97304 118.95328) (width 0.3048) (layer F.Cu) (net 17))
 (segment (start 155.26004 124.16536) (end 155.26004 107.85348) (width 0.3048) (layer F.Cu) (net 15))
 (segment (start 155.26004 124.16536) (end 152.89276 126.53264) (width 0.3048) (layer F.Cu) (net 15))
 (segment (start 152.89276 126.53264) (end 151.83612 126.53264) (width 0.3048) (layer F.Cu) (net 15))
 (segment (start 149.39772 124.09424) (end 151.83612 126.53264) (width 0.3048) (layer F.Cu) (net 15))
 (segment (start 150.60676 88.15832) (end 150.60676 85.73008) (width 0.3048) (layer F.Cu) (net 15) (status 800000))
 (segment (start 152.38476 89.93632) (end 150.60676 88.15832) (width 0.3048) (layer F.Cu) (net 15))
 (segment (start 152.38476 96.71812) (end 152.38476 89.93632) (width 0.3048) (layer F.Cu) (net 15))
 (segment (start 151.06904 98.03384) (end 152.38476 96.71812) (width 0.3048) (layer F.Cu) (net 15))
 (segment (start 151.06904 106.06024) (end 151.06904 98.03384) (width 0.3048) (layer F.Cu) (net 15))
 (segment (start 151.14016 106.13136) (end 151.06904 106.06024) (width 0.3048) (layer F.Cu) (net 15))
 (via (at 151.14016 106.13136) (size 0.889) (drill 0.635) (layers F.Cu B.Cu) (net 15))
 (segment (start 151.14016 106.19232) (end 151.14016 106.13136) (width 0.3048) (layer B.Cu) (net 15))
 (segment (start 152.21712 107.26928) (end 151.14016 106.19232) (width 0.3048) (layer B.Cu) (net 15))
 (segment (start 154.59456 107.26928) (end 152.21712 107.26928) (width 0.3048) (layer B.Cu) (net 15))
 (segment (start 155.20416 107.87888) (end 154.59456 107.26928) (width 0.3048) (layer B.Cu) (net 15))
 (via (at 155.20416 107.87888) (size 0.889) (drill 0.635) (layers F.Cu B.Cu) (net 15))
 (segment (start 155.23464 107.87888) (end 155.20416 107.87888) (width 0.3048) (layer F.Cu) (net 15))
 (segment (start 155.26004 107.85348) (end 155.23464 107.87888) (width 0.3048) (layer F.Cu) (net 15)))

